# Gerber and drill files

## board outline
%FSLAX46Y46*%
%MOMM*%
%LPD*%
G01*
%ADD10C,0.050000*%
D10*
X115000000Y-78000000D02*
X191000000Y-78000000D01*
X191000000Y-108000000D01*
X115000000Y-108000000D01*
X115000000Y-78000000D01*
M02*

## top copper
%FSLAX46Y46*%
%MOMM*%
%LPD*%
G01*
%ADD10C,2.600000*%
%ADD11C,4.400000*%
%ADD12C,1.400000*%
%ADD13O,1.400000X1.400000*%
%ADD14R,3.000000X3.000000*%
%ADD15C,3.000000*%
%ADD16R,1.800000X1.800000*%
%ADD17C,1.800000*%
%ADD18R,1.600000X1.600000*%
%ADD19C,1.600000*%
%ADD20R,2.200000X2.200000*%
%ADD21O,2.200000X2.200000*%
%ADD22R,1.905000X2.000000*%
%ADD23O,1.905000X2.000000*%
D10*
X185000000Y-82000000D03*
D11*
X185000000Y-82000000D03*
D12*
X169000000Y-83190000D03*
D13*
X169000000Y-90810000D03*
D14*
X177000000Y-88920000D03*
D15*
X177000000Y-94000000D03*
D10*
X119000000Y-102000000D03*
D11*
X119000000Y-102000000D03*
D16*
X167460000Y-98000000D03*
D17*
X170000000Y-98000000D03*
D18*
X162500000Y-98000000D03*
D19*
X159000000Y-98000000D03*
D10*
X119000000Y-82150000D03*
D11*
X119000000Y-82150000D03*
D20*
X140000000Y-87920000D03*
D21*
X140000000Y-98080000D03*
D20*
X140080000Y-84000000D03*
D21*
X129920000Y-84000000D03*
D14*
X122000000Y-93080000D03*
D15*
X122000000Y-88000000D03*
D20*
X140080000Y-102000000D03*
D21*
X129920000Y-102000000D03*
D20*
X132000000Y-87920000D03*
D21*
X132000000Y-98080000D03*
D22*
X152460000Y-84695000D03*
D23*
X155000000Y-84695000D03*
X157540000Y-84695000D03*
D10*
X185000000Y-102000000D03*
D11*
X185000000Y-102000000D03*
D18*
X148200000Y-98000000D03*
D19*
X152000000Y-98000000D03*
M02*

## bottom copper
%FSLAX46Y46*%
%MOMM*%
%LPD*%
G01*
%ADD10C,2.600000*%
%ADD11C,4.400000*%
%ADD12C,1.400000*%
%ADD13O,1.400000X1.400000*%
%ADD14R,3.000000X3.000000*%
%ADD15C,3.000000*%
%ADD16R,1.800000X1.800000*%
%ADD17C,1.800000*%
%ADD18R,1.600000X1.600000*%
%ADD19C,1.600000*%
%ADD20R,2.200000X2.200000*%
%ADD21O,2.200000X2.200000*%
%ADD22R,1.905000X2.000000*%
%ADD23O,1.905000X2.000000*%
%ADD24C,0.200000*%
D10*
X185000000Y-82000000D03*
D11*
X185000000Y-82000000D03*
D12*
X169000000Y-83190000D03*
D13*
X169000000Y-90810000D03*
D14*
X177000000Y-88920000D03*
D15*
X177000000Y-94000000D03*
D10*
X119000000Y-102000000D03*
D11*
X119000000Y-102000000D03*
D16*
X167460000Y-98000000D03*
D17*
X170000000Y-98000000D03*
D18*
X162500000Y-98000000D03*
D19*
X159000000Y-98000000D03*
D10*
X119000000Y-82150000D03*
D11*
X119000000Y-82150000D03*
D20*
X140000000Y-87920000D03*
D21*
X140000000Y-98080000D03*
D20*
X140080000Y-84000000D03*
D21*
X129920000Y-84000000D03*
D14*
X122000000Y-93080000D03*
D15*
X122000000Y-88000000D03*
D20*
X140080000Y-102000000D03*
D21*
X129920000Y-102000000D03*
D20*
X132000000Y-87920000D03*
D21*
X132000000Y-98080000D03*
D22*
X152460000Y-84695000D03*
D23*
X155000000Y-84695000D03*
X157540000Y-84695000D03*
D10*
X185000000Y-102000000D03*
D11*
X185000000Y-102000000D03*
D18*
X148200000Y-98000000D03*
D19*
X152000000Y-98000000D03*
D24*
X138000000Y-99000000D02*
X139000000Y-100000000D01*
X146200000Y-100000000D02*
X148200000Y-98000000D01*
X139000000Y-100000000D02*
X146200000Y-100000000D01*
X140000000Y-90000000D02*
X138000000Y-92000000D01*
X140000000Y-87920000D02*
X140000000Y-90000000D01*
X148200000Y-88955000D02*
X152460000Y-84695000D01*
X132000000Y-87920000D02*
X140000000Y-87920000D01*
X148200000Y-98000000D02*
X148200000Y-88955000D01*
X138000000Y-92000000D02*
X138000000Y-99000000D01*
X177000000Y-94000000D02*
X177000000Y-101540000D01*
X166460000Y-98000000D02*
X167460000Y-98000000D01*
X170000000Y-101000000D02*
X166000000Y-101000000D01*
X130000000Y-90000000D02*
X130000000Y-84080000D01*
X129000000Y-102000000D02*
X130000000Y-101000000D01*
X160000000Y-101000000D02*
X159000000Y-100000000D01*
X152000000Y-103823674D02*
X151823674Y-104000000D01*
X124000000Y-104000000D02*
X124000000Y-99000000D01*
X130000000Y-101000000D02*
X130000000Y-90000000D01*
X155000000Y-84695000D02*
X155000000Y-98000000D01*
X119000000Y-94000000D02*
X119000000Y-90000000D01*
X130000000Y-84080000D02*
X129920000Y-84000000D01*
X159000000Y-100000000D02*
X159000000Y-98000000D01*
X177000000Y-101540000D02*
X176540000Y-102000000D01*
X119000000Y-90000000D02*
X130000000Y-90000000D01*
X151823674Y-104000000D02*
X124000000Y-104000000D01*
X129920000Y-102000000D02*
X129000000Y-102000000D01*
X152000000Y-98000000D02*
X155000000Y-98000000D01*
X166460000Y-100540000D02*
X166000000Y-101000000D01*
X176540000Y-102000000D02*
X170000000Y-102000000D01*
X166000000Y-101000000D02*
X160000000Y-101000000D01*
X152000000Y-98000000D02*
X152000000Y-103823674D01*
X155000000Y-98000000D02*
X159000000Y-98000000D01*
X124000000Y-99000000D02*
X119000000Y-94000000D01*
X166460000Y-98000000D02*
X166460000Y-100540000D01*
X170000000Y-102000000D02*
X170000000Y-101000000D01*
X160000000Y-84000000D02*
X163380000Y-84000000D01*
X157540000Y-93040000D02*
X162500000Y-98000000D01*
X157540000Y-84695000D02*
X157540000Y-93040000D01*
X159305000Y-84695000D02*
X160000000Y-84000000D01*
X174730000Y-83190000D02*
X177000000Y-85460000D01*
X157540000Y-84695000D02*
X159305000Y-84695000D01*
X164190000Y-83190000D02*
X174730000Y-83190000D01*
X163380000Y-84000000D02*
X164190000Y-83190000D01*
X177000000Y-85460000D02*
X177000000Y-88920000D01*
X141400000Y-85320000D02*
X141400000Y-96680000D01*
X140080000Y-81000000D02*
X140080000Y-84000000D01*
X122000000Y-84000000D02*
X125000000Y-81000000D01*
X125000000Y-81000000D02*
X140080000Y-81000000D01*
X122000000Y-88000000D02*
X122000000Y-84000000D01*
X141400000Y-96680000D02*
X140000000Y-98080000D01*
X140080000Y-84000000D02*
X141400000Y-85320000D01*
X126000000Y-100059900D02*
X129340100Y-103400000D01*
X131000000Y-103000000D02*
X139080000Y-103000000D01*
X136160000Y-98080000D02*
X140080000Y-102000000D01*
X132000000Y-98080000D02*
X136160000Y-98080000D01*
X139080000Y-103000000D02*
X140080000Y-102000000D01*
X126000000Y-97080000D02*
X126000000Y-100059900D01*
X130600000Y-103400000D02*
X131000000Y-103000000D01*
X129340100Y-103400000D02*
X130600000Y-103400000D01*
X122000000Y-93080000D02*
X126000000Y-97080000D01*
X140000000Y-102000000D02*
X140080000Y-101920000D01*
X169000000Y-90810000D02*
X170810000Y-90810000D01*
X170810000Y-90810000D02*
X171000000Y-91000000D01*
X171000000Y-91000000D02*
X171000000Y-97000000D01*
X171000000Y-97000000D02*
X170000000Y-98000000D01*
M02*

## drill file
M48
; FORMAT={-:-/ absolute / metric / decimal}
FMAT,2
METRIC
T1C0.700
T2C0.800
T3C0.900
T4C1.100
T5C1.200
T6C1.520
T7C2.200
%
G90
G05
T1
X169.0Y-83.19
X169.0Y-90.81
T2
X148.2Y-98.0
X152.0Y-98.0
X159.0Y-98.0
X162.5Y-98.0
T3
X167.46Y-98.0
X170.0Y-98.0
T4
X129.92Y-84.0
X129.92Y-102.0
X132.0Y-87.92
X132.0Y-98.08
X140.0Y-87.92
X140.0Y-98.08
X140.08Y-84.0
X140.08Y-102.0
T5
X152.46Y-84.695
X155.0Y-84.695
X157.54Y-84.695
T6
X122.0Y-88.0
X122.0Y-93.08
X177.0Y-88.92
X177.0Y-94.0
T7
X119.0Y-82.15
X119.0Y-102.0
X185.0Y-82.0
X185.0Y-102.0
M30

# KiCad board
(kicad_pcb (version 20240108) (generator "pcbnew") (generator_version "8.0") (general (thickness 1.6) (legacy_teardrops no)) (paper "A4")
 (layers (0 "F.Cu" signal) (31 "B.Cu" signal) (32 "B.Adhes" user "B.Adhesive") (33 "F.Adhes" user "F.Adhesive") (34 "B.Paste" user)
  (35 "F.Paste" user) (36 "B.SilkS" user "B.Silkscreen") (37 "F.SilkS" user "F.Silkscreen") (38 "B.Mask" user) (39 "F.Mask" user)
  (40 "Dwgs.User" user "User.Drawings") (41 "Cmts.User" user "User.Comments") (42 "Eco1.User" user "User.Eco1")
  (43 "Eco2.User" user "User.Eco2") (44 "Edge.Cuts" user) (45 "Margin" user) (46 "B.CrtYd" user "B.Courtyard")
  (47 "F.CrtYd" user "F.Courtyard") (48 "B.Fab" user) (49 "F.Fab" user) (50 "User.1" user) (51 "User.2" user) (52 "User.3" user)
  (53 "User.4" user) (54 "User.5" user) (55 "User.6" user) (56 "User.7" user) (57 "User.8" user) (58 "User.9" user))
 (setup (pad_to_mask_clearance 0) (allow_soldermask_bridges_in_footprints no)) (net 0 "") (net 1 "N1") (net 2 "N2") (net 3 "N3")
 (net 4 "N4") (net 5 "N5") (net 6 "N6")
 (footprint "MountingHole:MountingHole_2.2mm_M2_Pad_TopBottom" (layer "F.Cu") (at 185 82)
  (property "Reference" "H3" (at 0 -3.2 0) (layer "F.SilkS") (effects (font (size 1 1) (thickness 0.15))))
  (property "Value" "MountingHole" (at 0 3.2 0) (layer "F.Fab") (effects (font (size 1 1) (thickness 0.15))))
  (pad "1" thru_hole circle (at 0 0) (size 2.6 2.6) (drill 2.2) (layers "*.Cu" "*.Mask") (remove_unused_layers no))
  (pad "1" connect circle (at 0 0) (size 4.4 4.4) (layers "F.Cu" "F.Mask"))
  (pad "1" connect circle (at 0 0) (size 4.4 4.4) (layers "B.Cu" "B.Mask")))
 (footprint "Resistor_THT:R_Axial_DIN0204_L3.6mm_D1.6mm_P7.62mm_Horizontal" (layer "F.Cu") (at 169 83.19 -90)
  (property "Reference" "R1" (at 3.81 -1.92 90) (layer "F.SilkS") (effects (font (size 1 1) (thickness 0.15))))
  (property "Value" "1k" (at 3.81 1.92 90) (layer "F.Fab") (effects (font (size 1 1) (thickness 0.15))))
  (pad "1" thru_hole circle (at 0 0 270) (size 1.4 1.4) (drill 0.7) (layers "*.Cu" "*.Mask") (remove_unused_layers no) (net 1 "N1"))
  (pad "2" thru_hole oval (at 7.62 0 270) (size 1.4 1.4) (drill 0.7) (layers "*.Cu" "*.Mask") (remove_unused_layers no) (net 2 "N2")))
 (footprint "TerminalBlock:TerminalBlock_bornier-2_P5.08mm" (layer "F.Cu") (at 177 88.92 -90)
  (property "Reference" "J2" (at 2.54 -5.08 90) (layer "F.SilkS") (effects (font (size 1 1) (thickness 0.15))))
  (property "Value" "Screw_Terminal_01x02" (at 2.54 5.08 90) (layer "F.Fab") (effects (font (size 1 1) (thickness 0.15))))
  (pad "1" thru_hole rect (at 0 0 270) (size 3 3) (drill 1.52) (layers "*.Cu" "*.Mask") (remove_unused_layers no) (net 1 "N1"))
  (pad "2" thru_hole circle (at 5.08 0 270) (size 3 3) (drill 1.52) (layers "*.Cu" "*.Mask") (remove_unused_layers no) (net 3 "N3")))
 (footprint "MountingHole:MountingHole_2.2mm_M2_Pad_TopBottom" (layer "F.Cu") (at 119 102)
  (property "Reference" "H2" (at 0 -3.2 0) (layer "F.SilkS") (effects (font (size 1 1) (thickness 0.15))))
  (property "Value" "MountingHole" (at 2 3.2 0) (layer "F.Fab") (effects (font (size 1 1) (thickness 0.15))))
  (pad "1" thru_hole circle (at 0 0) (size 2.6 2.6) (drill 2.2) (layers "*.Cu" "*.Mask") (remove_unused_layers no))
  (pad "1" connect circle (at 0 0) (size 4.4 4.4) (layers "F.Cu" "F.Mask"))
  (pad "1" connect circle (at 0 0) (size 4.4 4.4) (layers "B.Cu" "B.Mask")))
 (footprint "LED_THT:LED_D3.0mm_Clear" (layer "F.Cu") (at 167.46 98)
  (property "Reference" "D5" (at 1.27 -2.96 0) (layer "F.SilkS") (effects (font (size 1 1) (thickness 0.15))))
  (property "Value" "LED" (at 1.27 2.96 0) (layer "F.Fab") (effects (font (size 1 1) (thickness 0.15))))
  (pad "1" thru_hole rect (at 0 0) (size 1.8 1.8) (drill 0.9) (layers "*.Cu" "*.Mask") (remove_unused_layers no) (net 3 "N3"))
  (pad "2" thru_hole circle (at 2.54 0) (size 1.8 1.8) (drill 0.9) (layers "*.Cu" "*.Mask") (remove_unused_layers no) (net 2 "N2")))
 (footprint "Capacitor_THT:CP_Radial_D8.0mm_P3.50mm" (layer "F.Cu") (at 162.5 98 180)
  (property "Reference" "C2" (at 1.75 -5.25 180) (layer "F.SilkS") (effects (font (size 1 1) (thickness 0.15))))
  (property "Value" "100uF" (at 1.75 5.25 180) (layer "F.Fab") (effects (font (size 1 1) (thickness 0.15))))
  (pad "1" thru_hole rect (at 0 0 180) (size 1.6 1.6) (drill 0.8) (layers "*.Cu" "*.Mask") (remove_unused_layers no) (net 1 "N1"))
  (pad "2" thru_hole circle (at 3.5 0 180) (size 1.6 1.6) (drill 0.8) (layers "*.Cu" "*.Mask") (remove_unused_layers no) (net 3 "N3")))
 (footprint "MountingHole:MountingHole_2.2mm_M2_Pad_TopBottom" (layer "F.Cu") (at 119 82.15)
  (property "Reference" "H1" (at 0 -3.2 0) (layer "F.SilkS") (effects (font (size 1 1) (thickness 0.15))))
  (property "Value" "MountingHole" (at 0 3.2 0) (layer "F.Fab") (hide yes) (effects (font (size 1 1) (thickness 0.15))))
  (pad "1" thru_hole circle (at 0 0) (size 2.6 2.6) (drill 2.2) (layers "*.Cu" "*.Mask") (remove_unused_layers no))
  (pad "1" connect circle (at 0 0) (size 4.4 4.4) (layers "F.Cu" "F.Mask"))
  (pad "1" connect circle (at 0 0) (size 4.4 4.4) (layers "B.Cu" "B.Mask")))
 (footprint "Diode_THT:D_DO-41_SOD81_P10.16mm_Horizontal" (layer "F.Cu") (at 140 87.92 -90)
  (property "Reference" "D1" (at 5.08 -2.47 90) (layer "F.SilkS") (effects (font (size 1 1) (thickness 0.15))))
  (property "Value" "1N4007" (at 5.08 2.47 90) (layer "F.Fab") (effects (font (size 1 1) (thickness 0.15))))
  (pad "1" thru_hole rect (at 0 0 270) (size 2.2 2.2) (drill 1.1) (layers "*.Cu" "*.Mask") (remove_unused_layers no) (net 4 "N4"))
  (pad "2" thru_hole oval (at 10.16 0 270) (size 2.2 2.2) (drill 1.1) (layers "*.Cu" "*.Mask") (remove_unused_layers no) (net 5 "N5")))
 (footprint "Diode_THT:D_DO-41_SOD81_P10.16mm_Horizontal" (layer "F.Cu") (at 140.08 84 180)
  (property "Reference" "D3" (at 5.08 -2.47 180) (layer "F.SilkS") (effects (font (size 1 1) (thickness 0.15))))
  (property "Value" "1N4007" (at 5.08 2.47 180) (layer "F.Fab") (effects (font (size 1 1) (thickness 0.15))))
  (pad "1" thru_hole rect (at 0 0 180) (size 2.2 2.2) (drill 1.1) (layers "*.Cu" "*.Mask") (remove_unused_layers no) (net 5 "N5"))
  (pad "2" thru_hole oval (at 10.16 0 180) (size 2.2 2.2) (drill 1.1) (layers "*.Cu" "*.Mask") (remove_unused_layers no) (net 3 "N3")))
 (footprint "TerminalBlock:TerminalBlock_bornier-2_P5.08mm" (layer "F.Cu") (at 122 93.08 90)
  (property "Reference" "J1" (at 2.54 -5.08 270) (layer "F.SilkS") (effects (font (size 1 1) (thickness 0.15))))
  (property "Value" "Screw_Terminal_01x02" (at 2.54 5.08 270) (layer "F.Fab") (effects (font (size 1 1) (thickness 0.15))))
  (pad "1" thru_hole rect (at 0 0 90) (size 3 3) (drill 1.52) (layers "*.Cu" "*.Mask") (remove_unused_layers no) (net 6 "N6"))
  (pad "2" thru_hole circle (at 5.08 0 90) (size 3 3) (drill 1.52) (layers "*.Cu" "*.Mask") (remove_unused_layers no) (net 5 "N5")))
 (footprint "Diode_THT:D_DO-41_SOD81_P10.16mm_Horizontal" (layer "F.Cu") (at 140.08 102 180)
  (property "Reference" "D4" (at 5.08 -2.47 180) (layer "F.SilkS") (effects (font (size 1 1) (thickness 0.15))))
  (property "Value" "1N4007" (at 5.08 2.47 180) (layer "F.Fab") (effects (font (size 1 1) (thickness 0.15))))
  (pad "1" thru_hole rect (at 0 0 180) (size 2.2 2.2) (drill 1.1) (layers "*.Cu" "*.Mask") (remove_unused_layers no) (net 6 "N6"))
  (pad "2" thru_hole oval (at 10.16 0 180) (size 2.2 2.2) (drill 1.1) (layers "*.Cu" "*.Mask") (remove_unused_layers no) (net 3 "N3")))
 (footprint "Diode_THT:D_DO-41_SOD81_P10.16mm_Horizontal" (layer "F.Cu") (at 132 87.92 -90)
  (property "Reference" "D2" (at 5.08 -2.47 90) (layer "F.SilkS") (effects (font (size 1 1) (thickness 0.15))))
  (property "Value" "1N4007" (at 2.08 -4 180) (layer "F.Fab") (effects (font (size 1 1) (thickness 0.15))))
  (pad "1" thru_hole rect (at 0 0 270) (size 2.2 2.2) (drill 1.1) (layers "*.Cu" "*.Mask") (remove_unused_layers no) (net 4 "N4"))
  (pad "2" thru_hole oval (at 10.16 0 270) (size 2.2 2.2) (drill 1.1) (layers "*.Cu" "*.Mask") (remove_unused_layers no) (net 6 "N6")))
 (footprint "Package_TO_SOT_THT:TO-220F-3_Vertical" (layer "F.Cu") (at 152.46 84.695)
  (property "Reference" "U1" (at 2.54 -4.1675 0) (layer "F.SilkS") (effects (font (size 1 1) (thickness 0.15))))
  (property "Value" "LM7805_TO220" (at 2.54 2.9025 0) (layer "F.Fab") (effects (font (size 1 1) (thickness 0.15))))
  (pad "1" thru_hole rect (at 0 0) (size 1.905 2) (drill 1.2) (layers "*.Cu" "*.Mask") (remove_unused_layers no) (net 4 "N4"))
  (pad "2" thru_hole oval (at 2.54 0) (size 1.905 2) (drill 1.2) (layers "*.Cu" "*.Mask") (remove_unused_layers no) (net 3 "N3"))
  (pad "3" thru_hole oval (at 5.08 0) (size 1.905 2) (drill 1.2) (layers "*.Cu" "*.Mask") (remove_unused_layers no) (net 1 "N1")))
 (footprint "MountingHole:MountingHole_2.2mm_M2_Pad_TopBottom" (layer "F.Cu") (at 185 102)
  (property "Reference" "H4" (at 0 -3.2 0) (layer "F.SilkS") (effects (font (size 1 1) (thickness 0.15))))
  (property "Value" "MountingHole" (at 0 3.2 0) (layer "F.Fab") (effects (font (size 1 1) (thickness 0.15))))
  (pad "1" thru_hole circle (at 0 0) (size 2.6 2.6) (drill 2.2) (layers "*.Cu" "*.Mask") (remove_unused_layers no))
  (pad "1" connect circle (at 0 0) (size 4.4 4.4) (layers "F.Cu" "F.Mask"))
  (pad "1" connect circle (at 0 0) (size 4.4 4.4) (layers "B.Cu" "B.Mask")))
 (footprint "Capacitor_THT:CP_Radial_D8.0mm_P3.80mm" (layer "F.Cu") (at 148.2 98)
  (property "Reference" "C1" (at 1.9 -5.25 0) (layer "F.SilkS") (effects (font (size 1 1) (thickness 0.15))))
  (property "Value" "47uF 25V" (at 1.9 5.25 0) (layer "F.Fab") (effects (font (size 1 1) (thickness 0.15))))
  (pad "1" thru_hole rect (at 0 0) (size 1.6 1.6) (drill 0.8) (layers "*.Cu" "*.Mask") (remove_unused_layers no) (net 4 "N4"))
  (pad "2" thru_hole circle (at 3.8 0) (size 1.6 1.6) (drill 0.8) (layers "*.Cu" "*.Mask") (remove_unused_layers no) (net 3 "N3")))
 (gr_rect (start 115 78) (end 191 108) (stroke (width 0.05) (type default)) (fill none) (layer "Edge.Cuts"))
 (segment (start 138 99) (end 139 100) (width 0.2) (layer "B.Cu") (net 4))
 (segment (start 146.2 100) (end 148.2 98) (width 0.2) (layer "B.Cu") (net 4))
 (segment (start 139 100) (end 146.2 100) (width 0.2) (layer "B.Cu") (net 4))
 (segment (start 140 90) (end 138 92) (width 0.2) (layer "B.Cu") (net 4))
 (segment (start 140 87.92) (end 140 90) (width 0.2) (layer "B.Cu") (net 4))
 (segment (start 148.2 88.955) (end 152.46 84.695) (width 0.2) (layer "B.Cu") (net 4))
 (segment (start 132 87.92) (end 140 87.92) (width 0.2) (layer "B.Cu") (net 4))
 (segment (start 148.2 98) (end 148.2 88.955) (width 0.2) (layer "B.Cu") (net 4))
 (segment (start 138 92) (end 138 99) (width 0.2) (layer "B.Cu") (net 4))
 (segment (start 177 94) (end 177 101.54) (width 0.2) (layer "B.Cu") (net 3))
 (segment (start 166.46 98) (end 167.46 98) (width 0.2) (layer "B.Cu") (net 3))
 (segment (start 170 101) (end 166 101) (width 0.2) (layer "B.Cu") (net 3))
 (segment (start 130 90) (end 130 84.08) (width 0.2) (layer "B.Cu") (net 3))
 (segment (start 129 102) (end 130 101) (width 0.2) (layer "B.Cu") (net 3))
 (segment (start 160 101) (end 159 100) (width 0.2) (layer "B.Cu") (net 3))
 (segment (start 152 103.823674) (end 151.823674 104) (width 0.2) (layer "B.Cu") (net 3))
 (segment (start 124 104) (end 124 99) (width 0.2) (layer "B.Cu") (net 3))
 (segment (start 130 101) (end 130 90) (width 0.2) (layer "B.Cu") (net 3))
 (segment (start 155 84.695) (end 155 98) (width 0.2) (layer "B.Cu") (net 3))
 (segment (start 119 94) (end 119 90) (width 0.2) (layer "B.Cu") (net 3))
 (segment (start 130 84.08) (end 129.92 84) (width 0.2) (layer "B.Cu") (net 3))
 (segment (start 159 100) (end 159 98) (width 0.2) (layer "B.Cu") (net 3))
 (segment (start 177 101.54) (end 176.54 102) (width 0.2) (layer "B.Cu") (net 3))
 (segment (start 119 90) (end 130 90) (width 0.2) (layer "B.Cu") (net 3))
 (segment (start 151.823674 104) (end 124 104) (width 0.2) (layer "B.Cu") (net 3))
 (segment (start 129.92 102) (end 129 102) (width 0.2) (layer "B.Cu") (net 3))
 (segment (start 152 98) (end 155 98) (width 0.2) (layer "B.Cu") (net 3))
 (segment (start 166.46 100.54) (end 166 101) (width 0.2) (layer "B.Cu") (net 3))
 (segment (start 176.54 102) (end 170 102) (width 0.2) (layer "B.Cu") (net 3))
 (segment (start 166 101) (end 160 101) (width 0.2) (layer "B.Cu") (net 3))
 (segment (start 152 98) (end 152 103.823674) (width 0.2) (layer "B.Cu") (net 3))
 (segment (start 155 98) (end 159 98) (width 0.2) (layer "B.Cu") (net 3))
 (segment (start 124 99) (end 119 94) (width 0.2) (layer "B.Cu") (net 3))
 (segment (start 166.46 98) (end 166.46 100.54) (width 0.2) (layer "B.Cu") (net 3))
 (segment (start 170 102) (end 170 101) (width 0.2) (layer "B.Cu") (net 3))
 (segment (start 160 84) (end 163.38 84) (width 0.2) (layer "B.Cu") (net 1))
 (segment (start 157.54 93.04) (end 162.5 98) (width 0.2) (layer "B.Cu") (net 1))
 (segment (start 157.54 84.695) (end 157.54 93.04) (width 0.2) (layer "B.Cu") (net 1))
 (segment (start 159.305 84.695) (end 160 84) (width 0.2) (layer "B.Cu") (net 1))
 (segment (start 174.73 83.19) (end 177 85.46) (width 0.2) (layer "B.Cu") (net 1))
 (segment (start 157.54 84.695) (end 159.305 84.695) (width 0.2) (layer "B.Cu") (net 1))
 (segment (start 164.19 83.19) (end 174.73 83.19) (width 0.2) (layer "B.Cu") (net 1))
 (segment (start 163.38 84) (end 164.19 83.19) (width 0.2) (layer "B.Cu") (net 1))
 (segment (start 177 85.46) (end 177 88.92) (width 0.2) (layer "B.Cu") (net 1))
 (segment (start 141.4 85.32) (end 141.4 96.68) (width 0.2) (layer "B.Cu") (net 5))
 (segment (start 140.08 81) (end 140.08 84) (width 0.2) (layer "B.Cu") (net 5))
 (segment (start 122 84) (end 125 81) (width 0.2) (layer "B.Cu") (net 5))
 (segment (start 125 81) (end 140.08 81) (width 0.2) (layer "B.Cu") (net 5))
 (segment (start 122 88) (end 122 84) (width 0.2) (layer "B.Cu") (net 5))
 (segment (start 141.4 96.68) (end 140 98.08) (width 0.2) (layer "B.Cu") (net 5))
 (segment (start 140.08 84) (end 141.4 85.32) (width 0.2) (layer "B.Cu") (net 5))
 (segment (start 126 100.0599) (end 129.3401 103.4) (width 0.2) (layer "B.Cu") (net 6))
 (segment (start 131 103) (end 139.08 103) (width 0.2) (layer "B.Cu") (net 6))
 (segment (start 136.16 98.08) (end 140.08 102) (width 0.2) (layer "B.Cu") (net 6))
 (segment (start 132 98.08) (end 136.16 98.08) (width 0.2) (layer "B.Cu") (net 6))
 (segment (start 139.08 103) (end 140.08 102) (width 0.2) (layer "B.Cu") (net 6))
 (segment (start 126 97.08) (end 126 100.0599) (width 0.2) (layer "B.Cu") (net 6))
 (segment (start 130.6 103.4) (end 131 103) (width 0.2) (layer "B.Cu") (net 6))
 (segment (start 129.3401 103.4) (end 130.6 103.4) (width 0.2) (layer "B.Cu") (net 6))
 (segment (start 122 93.08) (end 126 97.08) (width 0.2) (layer "B.Cu") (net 6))
 (segment (start 140 102) (end 140.08 101.92) (width 0.2) (layer "B.Cu") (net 6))
 (segment (start 169 90.81) (end 170.81 90.81) (width 0.2) (layer "B.Cu") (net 2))
 (segment (start 170.81 90.81) (end 171 91) (width 0.2) (layer "B.Cu") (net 2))
 (segment (start 171 91) (end 171 97) (width 0.2) (layer "B.Cu") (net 2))
 (segment (start 171 97) (end 170 98) (width 0.2) (layer "B.Cu") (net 2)))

